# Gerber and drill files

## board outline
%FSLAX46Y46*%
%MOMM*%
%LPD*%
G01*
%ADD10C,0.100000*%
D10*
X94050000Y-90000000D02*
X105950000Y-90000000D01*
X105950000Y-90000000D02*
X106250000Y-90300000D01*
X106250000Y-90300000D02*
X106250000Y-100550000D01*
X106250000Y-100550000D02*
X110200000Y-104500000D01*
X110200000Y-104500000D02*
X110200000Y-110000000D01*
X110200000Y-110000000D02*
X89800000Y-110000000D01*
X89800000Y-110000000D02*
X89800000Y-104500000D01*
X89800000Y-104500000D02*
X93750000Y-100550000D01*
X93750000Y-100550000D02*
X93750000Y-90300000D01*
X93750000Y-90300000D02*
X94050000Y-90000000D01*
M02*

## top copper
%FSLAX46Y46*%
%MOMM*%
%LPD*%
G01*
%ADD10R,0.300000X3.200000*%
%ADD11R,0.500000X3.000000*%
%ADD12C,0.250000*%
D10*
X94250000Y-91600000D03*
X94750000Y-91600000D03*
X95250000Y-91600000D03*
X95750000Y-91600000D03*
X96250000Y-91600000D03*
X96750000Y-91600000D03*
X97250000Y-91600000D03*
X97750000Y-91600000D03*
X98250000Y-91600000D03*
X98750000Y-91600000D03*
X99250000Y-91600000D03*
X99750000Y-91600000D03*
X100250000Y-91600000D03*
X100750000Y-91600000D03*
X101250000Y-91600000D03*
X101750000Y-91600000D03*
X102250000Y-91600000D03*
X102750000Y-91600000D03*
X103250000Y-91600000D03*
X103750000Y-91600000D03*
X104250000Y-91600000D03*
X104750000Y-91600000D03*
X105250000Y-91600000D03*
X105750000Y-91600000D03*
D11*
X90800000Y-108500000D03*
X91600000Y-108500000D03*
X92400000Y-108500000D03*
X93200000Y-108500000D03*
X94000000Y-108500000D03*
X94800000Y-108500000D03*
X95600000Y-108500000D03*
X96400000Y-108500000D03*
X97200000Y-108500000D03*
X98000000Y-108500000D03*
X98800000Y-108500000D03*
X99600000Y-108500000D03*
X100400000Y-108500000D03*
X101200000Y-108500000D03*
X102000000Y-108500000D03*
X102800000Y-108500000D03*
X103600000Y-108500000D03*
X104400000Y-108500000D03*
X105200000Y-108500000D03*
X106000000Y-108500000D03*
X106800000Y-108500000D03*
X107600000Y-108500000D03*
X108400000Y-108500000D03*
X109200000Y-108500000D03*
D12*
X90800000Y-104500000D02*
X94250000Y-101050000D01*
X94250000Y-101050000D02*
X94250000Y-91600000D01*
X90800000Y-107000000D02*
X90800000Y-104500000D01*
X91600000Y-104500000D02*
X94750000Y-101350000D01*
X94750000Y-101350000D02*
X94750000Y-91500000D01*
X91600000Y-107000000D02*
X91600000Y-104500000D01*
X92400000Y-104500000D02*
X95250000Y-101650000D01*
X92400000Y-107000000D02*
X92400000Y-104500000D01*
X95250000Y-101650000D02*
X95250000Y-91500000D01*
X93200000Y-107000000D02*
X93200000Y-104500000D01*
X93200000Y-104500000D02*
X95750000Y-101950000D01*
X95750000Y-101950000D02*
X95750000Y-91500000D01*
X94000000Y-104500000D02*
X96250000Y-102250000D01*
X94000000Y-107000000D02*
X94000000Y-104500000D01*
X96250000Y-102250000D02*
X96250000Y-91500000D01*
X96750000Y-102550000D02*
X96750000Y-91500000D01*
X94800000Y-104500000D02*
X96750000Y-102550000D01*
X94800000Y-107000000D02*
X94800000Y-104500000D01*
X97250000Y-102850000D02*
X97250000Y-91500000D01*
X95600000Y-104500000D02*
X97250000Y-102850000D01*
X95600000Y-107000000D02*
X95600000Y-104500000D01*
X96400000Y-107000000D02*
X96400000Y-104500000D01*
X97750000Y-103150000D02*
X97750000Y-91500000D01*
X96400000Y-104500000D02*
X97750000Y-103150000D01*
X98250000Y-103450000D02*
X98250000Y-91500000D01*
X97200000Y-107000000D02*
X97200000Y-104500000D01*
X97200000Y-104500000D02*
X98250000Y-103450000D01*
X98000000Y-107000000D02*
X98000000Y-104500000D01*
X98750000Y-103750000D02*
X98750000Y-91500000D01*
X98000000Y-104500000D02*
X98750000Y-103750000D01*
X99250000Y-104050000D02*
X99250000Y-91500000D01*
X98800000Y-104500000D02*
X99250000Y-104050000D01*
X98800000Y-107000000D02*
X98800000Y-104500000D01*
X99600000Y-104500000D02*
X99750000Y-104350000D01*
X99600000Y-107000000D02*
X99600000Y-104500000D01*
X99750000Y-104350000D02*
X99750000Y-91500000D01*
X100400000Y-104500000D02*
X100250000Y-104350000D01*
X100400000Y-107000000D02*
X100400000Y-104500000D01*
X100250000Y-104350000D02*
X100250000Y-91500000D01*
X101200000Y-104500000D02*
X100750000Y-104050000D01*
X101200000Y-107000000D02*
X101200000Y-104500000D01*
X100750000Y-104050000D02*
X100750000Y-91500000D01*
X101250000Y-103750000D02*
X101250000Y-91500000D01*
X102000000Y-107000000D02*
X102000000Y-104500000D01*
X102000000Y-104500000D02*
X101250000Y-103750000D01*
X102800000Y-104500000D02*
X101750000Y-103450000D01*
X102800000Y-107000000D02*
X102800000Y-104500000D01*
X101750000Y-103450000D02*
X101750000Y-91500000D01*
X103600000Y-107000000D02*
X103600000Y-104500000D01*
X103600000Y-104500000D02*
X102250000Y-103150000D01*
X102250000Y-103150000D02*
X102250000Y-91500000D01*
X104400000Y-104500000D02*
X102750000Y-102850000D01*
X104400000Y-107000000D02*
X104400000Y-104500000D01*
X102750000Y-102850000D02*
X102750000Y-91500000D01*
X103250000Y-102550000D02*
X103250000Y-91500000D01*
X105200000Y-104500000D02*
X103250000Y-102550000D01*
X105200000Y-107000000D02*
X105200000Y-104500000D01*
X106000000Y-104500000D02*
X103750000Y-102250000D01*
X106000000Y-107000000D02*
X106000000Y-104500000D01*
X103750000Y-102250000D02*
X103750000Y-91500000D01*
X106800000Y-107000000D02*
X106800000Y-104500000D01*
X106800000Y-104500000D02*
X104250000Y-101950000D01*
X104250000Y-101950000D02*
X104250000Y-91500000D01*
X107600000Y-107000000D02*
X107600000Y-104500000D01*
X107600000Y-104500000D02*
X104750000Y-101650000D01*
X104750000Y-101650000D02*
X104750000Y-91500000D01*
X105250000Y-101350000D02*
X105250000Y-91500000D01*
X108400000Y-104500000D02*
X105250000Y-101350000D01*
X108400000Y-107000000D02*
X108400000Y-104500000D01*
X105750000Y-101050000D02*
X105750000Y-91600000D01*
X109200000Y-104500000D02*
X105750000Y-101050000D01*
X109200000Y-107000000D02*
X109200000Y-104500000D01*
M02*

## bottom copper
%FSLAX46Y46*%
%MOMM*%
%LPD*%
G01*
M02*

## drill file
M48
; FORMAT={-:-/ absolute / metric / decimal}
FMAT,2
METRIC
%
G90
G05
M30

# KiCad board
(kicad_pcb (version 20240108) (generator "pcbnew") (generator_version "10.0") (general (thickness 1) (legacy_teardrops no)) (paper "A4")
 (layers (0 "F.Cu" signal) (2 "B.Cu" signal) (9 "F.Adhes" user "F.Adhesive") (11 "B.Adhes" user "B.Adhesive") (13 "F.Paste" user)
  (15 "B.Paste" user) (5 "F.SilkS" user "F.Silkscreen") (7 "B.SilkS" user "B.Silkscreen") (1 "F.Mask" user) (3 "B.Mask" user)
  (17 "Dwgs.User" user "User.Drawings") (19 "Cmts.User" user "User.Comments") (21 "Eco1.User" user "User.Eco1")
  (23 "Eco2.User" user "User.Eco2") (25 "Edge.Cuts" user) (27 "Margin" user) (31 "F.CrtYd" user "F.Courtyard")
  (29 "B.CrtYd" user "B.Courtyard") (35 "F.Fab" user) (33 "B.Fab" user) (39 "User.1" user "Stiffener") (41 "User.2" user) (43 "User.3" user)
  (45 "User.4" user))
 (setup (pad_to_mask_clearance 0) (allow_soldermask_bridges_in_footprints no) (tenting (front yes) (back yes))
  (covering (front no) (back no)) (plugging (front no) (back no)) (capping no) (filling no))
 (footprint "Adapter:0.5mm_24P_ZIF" (layer "F.Cu") (at 100 91.6)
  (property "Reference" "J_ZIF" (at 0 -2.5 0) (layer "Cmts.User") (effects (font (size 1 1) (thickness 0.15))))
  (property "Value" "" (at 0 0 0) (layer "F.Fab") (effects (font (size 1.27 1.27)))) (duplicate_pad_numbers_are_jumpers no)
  (pad "1" smd rect (at -5.75 0) (size 0.3 3.2) (layers "F.Cu" "F.Paste") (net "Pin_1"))
  (pad "2" smd rect (at -5.25 0) (size 0.3 3.2) (layers "F.Cu" "F.Paste") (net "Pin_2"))
  (pad "3" smd rect (at -4.75 0) (size 0.3 3.2) (layers "F.Cu" "F.Paste") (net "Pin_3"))
  (pad "4" smd rect (at -4.25 0) (size 0.3 3.2) (layers "F.Cu" "F.Paste") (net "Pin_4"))
  (pad "5" smd rect (at -3.75 0) (size 0.3 3.2) (layers "F.Cu" "F.Paste") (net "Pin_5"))
  (pad "6" smd rect (at -3.25 0) (size 0.3 3.2) (layers "F.Cu" "F.Paste") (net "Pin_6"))
  (pad "7" smd rect (at -2.75 0) (size 0.3 3.2) (layers "F.Cu" "F.Paste") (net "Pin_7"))
  (pad "8" smd rect (at -2.25 0) (size 0.3 3.2) (layers "F.Cu" "F.Paste") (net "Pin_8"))
  (pad "9" smd rect (at -1.75 0) (size 0.3 3.2) (layers "F.Cu" "F.Paste") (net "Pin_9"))
  (pad "10" smd rect (at -1.25 0) (size 0.3 3.2) (layers "F.Cu" "F.Paste") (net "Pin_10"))
  (pad "11" smd rect (at -0.75 0) (size 0.3 3.2) (layers "F.Cu" "F.Paste") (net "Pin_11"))
  (pad "12" smd rect (at -0.25 0) (size 0.3 3.2) (layers "F.Cu" "F.Paste") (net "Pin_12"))
  (pad "13" smd rect (at 0.25 0) (size 0.3 3.2) (layers "F.Cu" "F.Paste") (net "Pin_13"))
  (pad "14" smd rect (at 0.75 0) (size 0.3 3.2) (layers "F.Cu" "F.Paste") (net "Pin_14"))
  (pad "15" smd rect (at 1.25 0) (size 0.3 3.2) (layers "F.Cu" "F.Paste") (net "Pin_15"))
  (pad "16" smd rect (at 1.75 0) (size 0.3 3.2) (layers "F.Cu" "F.Paste") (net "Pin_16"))
  (pad "17" smd rect (at 2.25 0) (size 0.3 3.2) (layers "F.Cu" "F.Paste") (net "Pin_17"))
  (pad "18" smd rect (at 2.75 0) (size 0.3 3.2) (layers "F.Cu" "F.Paste") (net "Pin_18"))
  (pad "19" smd rect (at 3.25 0) (size 0.3 3.2) (layers "F.Cu" "F.Paste") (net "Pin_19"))
  (pad "20" smd rect (at 3.75 0) (size 0.3 3.2) (layers "F.Cu" "F.Paste") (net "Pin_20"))
  (pad "21" smd rect (at 4.25 0) (size 0.3 3.2) (layers "F.Cu" "F.Paste") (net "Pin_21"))
  (pad "22" smd rect (at 4.75 0) (size 0.3 3.2) (layers "F.Cu" "F.Paste") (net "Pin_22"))
  (pad "23" smd rect (at 5.25 0) (size 0.3 3.2) (layers "F.Cu" "F.Paste") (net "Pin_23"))
  (pad "24" smd rect (at 5.75 0) (size 0.3 3.2) (layers "F.Cu" "F.Paste") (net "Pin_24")))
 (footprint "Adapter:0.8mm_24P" (layer "F.Cu") (at 100 108.5)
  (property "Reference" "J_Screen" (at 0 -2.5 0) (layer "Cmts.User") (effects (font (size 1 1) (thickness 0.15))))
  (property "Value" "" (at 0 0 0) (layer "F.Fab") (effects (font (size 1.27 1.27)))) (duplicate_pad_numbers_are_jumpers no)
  (pad "1" smd rect (at -9.20 0) (size 0.5 3) (layers "F.Cu" "F.Mask" "F.Paste") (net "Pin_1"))
  (pad "2" smd rect (at -8.40 0) (size 0.5 3) (layers "F.Cu" "F.Mask" "F.Paste") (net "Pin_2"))
  (pad "3" smd rect (at -7.60 0) (size 0.5 3) (layers "F.Cu" "F.Mask" "F.Paste") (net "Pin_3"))
  (pad "4" smd rect (at -6.80 0) (size 0.5 3) (layers "F.Cu" "F.Mask" "F.Paste") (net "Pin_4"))
  (pad "5" smd rect (at -6.00 0) (size 0.5 3) (layers "F.Cu" "F.Mask" "F.Paste") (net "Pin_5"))
  (pad "6" smd rect (at -5.20 0) (size 0.5 3) (layers "F.Cu" "F.Mask" "F.Paste") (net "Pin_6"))
  (pad "7" smd rect (at -4.40 0) (size 0.5 3) (layers "F.Cu" "F.Mask" "F.Paste") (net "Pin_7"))
  (pad "8" smd rect (at -3.60 0) (size 0.5 3) (layers "F.Cu" "F.Mask" "F.Paste") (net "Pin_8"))
  (pad "9" smd rect (at -2.80 0) (size 0.5 3) (layers "F.Cu" "F.Mask" "F.Paste") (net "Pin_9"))
  (pad "10" smd rect (at -2.00 0) (size 0.5 3) (layers "F.Cu" "F.Mask" "F.Paste") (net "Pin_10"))
  (pad "11" smd rect (at -1.20 0) (size 0.5 3) (layers "F.Cu" "F.Mask" "F.Paste") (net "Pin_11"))
  (pad "12" smd rect (at -0.40 0) (size 0.5 3) (layers "F.Cu" "F.Mask" "F.Paste") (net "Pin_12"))
  (pad "13" smd rect (at 0.40 0) (size 0.5 3) (layers "F.Cu" "F.Mask" "F.Paste") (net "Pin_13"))
  (pad "14" smd rect (at 1.20 0) (size 0.5 3) (layers "F.Cu" "F.Mask" "F.Paste") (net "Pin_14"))
  (pad "15" smd rect (at 2.00 0) (size 0.5 3) (layers "F.Cu" "F.Mask" "F.Paste") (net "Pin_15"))
  (pad "16" smd rect (at 2.80 0) (size 0.5 3) (layers "F.Cu" "F.Mask" "F.Paste") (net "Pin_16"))
  (pad "17" smd rect (at 3.60 0) (size 0.5 3) (layers "F.Cu" "F.Mask" "F.Paste") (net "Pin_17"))
  (pad "18" smd rect (at 4.40 0) (size 0.5 3) (layers "F.Cu" "F.Mask" "F.Paste") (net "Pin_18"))
  (pad "19" smd rect (at 5.20 0) (size 0.5 3) (layers "F.Cu" "F.Mask" "F.Paste") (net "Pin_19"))
  (pad "20" smd rect (at 6.00 0) (size 0.5 3) (layers "F.Cu" "F.Mask" "F.Paste") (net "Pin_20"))
  (pad "21" smd rect (at 6.80 0) (size 0.5 3) (layers "F.Cu" "F.Mask" "F.Paste") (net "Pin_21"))
  (pad "22" smd rect (at 7.60 0) (size 0.5 3) (layers "F.Cu" "F.Mask" "F.Paste") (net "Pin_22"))
  (pad "23" smd rect (at 8.40 0) (size 0.5 3) (layers "F.Cu" "F.Mask" "F.Paste") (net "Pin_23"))
  (pad "24" smd rect (at 9.20 0) (size 0.5 3) (layers "F.Cu" "F.Mask" "F.Paste") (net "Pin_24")))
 (segment (start 90.8 104.5) (end 94.25 101.05) (width 0.25) (layer "F.Cu") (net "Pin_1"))
 (segment (start 94.25 101.05) (end 94.25 91.6) (width 0.25) (layer "F.Cu") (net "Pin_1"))
 (segment (start 90.8 107) (end 90.8 104.5) (width 0.25) (layer "F.Cu") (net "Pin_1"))
 (segment (start 91.6 104.5) (end 94.75 101.35) (width 0.25) (layer "F.Cu") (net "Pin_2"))
 (segment (start 94.75 101.35) (end 94.75 91.5) (width 0.25) (layer "F.Cu") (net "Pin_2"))
 (segment (start 91.6 107) (end 91.6 104.5) (width 0.25) (layer "F.Cu") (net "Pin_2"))
 (segment (start 92.4 104.5) (end 95.25 101.65) (width 0.25) (layer "F.Cu") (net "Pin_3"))
 (segment (start 92.4 107) (end 92.4 104.5) (width 0.25) (layer "F.Cu") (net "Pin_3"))
 (segment (start 95.25 101.65) (end 95.25 91.5) (width 0.25) (layer "F.Cu") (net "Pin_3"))
 (segment (start 93.2 107) (end 93.2 104.5) (width 0.25) (layer "F.Cu") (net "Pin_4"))
 (segment (start 93.2 104.5) (end 95.75 101.95) (width 0.25) (layer "F.Cu") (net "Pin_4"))
 (segment (start 95.75 101.95) (end 95.75 91.5) (width 0.25) (layer "F.Cu") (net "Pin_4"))
 (segment (start 94 104.5) (end 96.25 102.25) (width 0.25) (layer "F.Cu") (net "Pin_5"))
 (segment (start 94 107) (end 94 104.5) (width 0.25) (layer "F.Cu") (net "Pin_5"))
 (segment (start 96.25 102.25) (end 96.25 91.5) (width 0.25) (layer "F.Cu") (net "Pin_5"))
 (segment (start 96.75 102.55) (end 96.75 91.5) (width 0.25) (layer "F.Cu") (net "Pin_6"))
 (segment (start 94.8 104.5) (end 96.75 102.55) (width 0.25) (layer "F.Cu") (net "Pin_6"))
 (segment (start 94.8 107) (end 94.8 104.5) (width 0.25) (layer "F.Cu") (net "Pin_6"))
 (segment (start 97.25 102.85) (end 97.25 91.5) (width 0.25) (layer "F.Cu") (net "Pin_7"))
 (segment (start 95.6 104.5) (end 97.25 102.85) (width 0.25) (layer "F.Cu") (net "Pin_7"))
 (segment (start 95.6 107) (end 95.6 104.5) (width 0.25) (layer "F.Cu") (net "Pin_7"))
 (segment (start 96.4 107) (end 96.4 104.5) (width 0.25) (layer "F.Cu") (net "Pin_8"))
 (segment (start 97.75 103.15) (end 97.75 91.5) (width 0.25) (layer "F.Cu") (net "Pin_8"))
 (segment (start 96.4 104.5) (end 97.75 103.15) (width 0.25) (layer "F.Cu") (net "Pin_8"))
 (segment (start 98.25 103.45) (end 98.25 91.5) (width 0.25) (layer "F.Cu") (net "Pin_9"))
 (segment (start 97.2 107) (end 97.2 104.5) (width 0.25) (layer "F.Cu") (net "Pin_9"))
 (segment (start 97.2 104.5) (end 98.25 103.45) (width 0.25) (layer "F.Cu") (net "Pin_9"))
 (segment (start 98 107) (end 98 104.5) (width 0.25) (layer "F.Cu") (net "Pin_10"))
 (segment (start 98.75 103.75) (end 98.75 91.5) (width 0.25) (layer "F.Cu") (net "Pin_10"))
 (segment (start 98 104.5) (end 98.75 103.75) (width 0.25) (layer "F.Cu") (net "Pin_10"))
 (segment (start 99.25 104.05) (end 99.25 91.5) (width 0.25) (layer "F.Cu") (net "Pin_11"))
 (segment (start 98.8 104.5) (end 99.25 104.05) (width 0.25) (layer "F.Cu") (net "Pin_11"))
 (segment (start 98.8 107) (end 98.8 104.5) (width 0.25) (layer "F.Cu") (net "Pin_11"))
 (segment (start 99.6 104.5) (end 99.75 104.35) (width 0.25) (layer "F.Cu") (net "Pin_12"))
 (segment (start 99.6 107) (end 99.6 104.5) (width 0.25) (layer "F.Cu") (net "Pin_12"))
 (segment (start 99.75 104.35) (end 99.75 91.5) (width 0.25) (layer "F.Cu") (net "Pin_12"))
 (segment (start 100.4 104.5) (end 100.25 104.35) (width 0.25) (layer "F.Cu") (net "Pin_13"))
 (segment (start 100.4 107) (end 100.4 104.5) (width 0.25) (layer "F.Cu") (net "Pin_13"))
 (segment (start 100.25 104.35) (end 100.25 91.5) (width 0.25) (layer "F.Cu") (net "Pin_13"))
 (segment (start 101.2 104.5) (end 100.75 104.05) (width 0.25) (layer "F.Cu") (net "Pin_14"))
 (segment (start 101.2 107) (end 101.2 104.5) (width 0.25) (layer "F.Cu") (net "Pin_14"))
 (segment (start 100.75 104.05) (end 100.75 91.5) (width 0.25) (layer "F.Cu") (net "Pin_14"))
 (segment (start 101.25 103.75) (end 101.25 91.5) (width 0.25) (layer "F.Cu") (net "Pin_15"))
 (segment (start 102 107) (end 102 104.5) (width 0.25) (layer "F.Cu") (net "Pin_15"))
 (segment (start 102 104.5) (end 101.25 103.75) (width 0.25) (layer "F.Cu") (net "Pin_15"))
 (segment (start 102.8 104.5) (end 101.75 103.45) (width 0.25) (layer "F.Cu") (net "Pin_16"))
 (segment (start 102.8 107) (end 102.8 104.5) (width 0.25) (layer "F.Cu") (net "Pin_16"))
 (segment (start 101.75 103.45) (end 101.75 91.5) (width 0.25) (layer "F.Cu") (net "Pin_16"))
 (segment (start 103.6 107) (end 103.6 104.5) (width 0.25) (layer "F.Cu") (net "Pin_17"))
 (segment (start 103.6 104.5) (end 102.25 103.15) (width 0.25) (layer "F.Cu") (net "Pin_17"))
 (segment (start 102.25 103.15) (end 102.25 91.5) (width 0.25) (layer "F.Cu") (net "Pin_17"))
 (segment (start 104.4 104.5) (end 102.75 102.85) (width 0.25) (layer "F.Cu") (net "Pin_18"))
 (segment (start 104.4 107) (end 104.4 104.5) (width 0.25) (layer "F.Cu") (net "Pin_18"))
 (segment (start 102.75 102.85) (end 102.75 91.5) (width 0.25) (layer "F.Cu") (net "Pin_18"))
 (segment (start 103.25 102.55) (end 103.25 91.5) (width 0.25) (layer "F.Cu") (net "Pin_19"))
 (segment (start 105.2 104.5) (end 103.25 102.55) (width 0.25) (layer "F.Cu") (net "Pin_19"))
 (segment (start 105.2 107) (end 105.2 104.5) (width 0.25) (layer "F.Cu") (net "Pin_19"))
 (segment (start 106 104.5) (end 103.75 102.25) (width 0.25) (layer "F.Cu") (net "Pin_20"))
 (segment (start 106 107) (end 106 104.5) (width 0.25) (layer "F.Cu") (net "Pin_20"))
 (segment (start 103.75 102.25) (end 103.75 91.5) (width 0.25) (layer "F.Cu") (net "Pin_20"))
 (segment (start 106.8 107) (end 106.8 104.5) (width 0.25) (layer "F.Cu") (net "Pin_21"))
 (segment (start 106.8 104.5) (end 104.25 101.95) (width 0.25) (layer "F.Cu") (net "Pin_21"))
 (segment (start 104.25 101.95) (end 104.25 91.5) (width 0.25) (layer "F.Cu") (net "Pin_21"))
 (segment (start 107.6 107) (end 107.6 104.5) (width 0.25) (layer "F.Cu") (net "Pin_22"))
 (segment (start 107.6 104.5) (end 104.75 101.65) (width 0.25) (layer "F.Cu") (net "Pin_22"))
 (segment (start 104.75 101.65) (end 104.75 91.5) (width 0.25) (layer "F.Cu") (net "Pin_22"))
 (segment (start 105.25 101.35) (end 105.25 91.5) (width 0.25) (layer "F.Cu") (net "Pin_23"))
 (segment (start 108.4 104.5) (end 105.25 101.35) (width 0.25) (layer "F.Cu") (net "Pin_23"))
 (segment (start 108.4 107) (end 108.4 104.5) (width 0.25) (layer "F.Cu") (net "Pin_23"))
 (segment (start 105.75 101.05) (end 105.75 91.6) (width 0.25) (layer "F.Cu") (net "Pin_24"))
 (segment (start 109.2 104.5) (end 105.75 101.05) (width 0.25) (layer "F.Cu") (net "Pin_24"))
 (segment (start 109.2 107) (end 109.2 104.5) (width 0.25) (layer "F.Cu") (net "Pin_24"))
 (gr_line (start 94.05 90.0) (end 105.95 90.0) (stroke (width 0.1) (type solid)) (layer "Edge.Cuts"))
 (gr_line (start 105.95 90.0) (end 106.25 90.3) (stroke (width 0.1) (type solid)) (layer "Edge.Cuts"))
 (gr_line (start 106.25 90.3) (end 106.25 100.55) (stroke (width 0.1) (type solid)) (layer "Edge.Cuts"))
 (gr_line (start 106.25 100.55) (end 110.2 104.5) (stroke (width 0.1) (type solid)) (layer "Edge.Cuts"))
 (gr_line (start 110.2 104.5) (end 110.2 110.0) (stroke (width 0.1) (type solid)) (layer "Edge.Cuts"))
 (gr_line (start 110.2 110.0) (end 89.8 110.0) (stroke (width 0.1) (type solid)) (layer "Edge.Cuts"))
 (gr_line (start 89.8 110.0) (end 89.8 104.5) (stroke (width 0.1) (type solid)) (layer "Edge.Cuts"))
 (gr_line (start 89.8 104.5) (end 93.75 100.55) (stroke (width 0.1) (type solid)) (layer "Edge.Cuts"))
 (gr_line (start 93.75 100.55) (end 93.75 90.3) (stroke (width 0.1) (type solid)) (layer "Edge.Cuts"))
 (gr_line (start 93.75 90.3) (end 94.05 90.0) (stroke (width 0.1) (type solid)) (layer "Edge.Cuts")))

